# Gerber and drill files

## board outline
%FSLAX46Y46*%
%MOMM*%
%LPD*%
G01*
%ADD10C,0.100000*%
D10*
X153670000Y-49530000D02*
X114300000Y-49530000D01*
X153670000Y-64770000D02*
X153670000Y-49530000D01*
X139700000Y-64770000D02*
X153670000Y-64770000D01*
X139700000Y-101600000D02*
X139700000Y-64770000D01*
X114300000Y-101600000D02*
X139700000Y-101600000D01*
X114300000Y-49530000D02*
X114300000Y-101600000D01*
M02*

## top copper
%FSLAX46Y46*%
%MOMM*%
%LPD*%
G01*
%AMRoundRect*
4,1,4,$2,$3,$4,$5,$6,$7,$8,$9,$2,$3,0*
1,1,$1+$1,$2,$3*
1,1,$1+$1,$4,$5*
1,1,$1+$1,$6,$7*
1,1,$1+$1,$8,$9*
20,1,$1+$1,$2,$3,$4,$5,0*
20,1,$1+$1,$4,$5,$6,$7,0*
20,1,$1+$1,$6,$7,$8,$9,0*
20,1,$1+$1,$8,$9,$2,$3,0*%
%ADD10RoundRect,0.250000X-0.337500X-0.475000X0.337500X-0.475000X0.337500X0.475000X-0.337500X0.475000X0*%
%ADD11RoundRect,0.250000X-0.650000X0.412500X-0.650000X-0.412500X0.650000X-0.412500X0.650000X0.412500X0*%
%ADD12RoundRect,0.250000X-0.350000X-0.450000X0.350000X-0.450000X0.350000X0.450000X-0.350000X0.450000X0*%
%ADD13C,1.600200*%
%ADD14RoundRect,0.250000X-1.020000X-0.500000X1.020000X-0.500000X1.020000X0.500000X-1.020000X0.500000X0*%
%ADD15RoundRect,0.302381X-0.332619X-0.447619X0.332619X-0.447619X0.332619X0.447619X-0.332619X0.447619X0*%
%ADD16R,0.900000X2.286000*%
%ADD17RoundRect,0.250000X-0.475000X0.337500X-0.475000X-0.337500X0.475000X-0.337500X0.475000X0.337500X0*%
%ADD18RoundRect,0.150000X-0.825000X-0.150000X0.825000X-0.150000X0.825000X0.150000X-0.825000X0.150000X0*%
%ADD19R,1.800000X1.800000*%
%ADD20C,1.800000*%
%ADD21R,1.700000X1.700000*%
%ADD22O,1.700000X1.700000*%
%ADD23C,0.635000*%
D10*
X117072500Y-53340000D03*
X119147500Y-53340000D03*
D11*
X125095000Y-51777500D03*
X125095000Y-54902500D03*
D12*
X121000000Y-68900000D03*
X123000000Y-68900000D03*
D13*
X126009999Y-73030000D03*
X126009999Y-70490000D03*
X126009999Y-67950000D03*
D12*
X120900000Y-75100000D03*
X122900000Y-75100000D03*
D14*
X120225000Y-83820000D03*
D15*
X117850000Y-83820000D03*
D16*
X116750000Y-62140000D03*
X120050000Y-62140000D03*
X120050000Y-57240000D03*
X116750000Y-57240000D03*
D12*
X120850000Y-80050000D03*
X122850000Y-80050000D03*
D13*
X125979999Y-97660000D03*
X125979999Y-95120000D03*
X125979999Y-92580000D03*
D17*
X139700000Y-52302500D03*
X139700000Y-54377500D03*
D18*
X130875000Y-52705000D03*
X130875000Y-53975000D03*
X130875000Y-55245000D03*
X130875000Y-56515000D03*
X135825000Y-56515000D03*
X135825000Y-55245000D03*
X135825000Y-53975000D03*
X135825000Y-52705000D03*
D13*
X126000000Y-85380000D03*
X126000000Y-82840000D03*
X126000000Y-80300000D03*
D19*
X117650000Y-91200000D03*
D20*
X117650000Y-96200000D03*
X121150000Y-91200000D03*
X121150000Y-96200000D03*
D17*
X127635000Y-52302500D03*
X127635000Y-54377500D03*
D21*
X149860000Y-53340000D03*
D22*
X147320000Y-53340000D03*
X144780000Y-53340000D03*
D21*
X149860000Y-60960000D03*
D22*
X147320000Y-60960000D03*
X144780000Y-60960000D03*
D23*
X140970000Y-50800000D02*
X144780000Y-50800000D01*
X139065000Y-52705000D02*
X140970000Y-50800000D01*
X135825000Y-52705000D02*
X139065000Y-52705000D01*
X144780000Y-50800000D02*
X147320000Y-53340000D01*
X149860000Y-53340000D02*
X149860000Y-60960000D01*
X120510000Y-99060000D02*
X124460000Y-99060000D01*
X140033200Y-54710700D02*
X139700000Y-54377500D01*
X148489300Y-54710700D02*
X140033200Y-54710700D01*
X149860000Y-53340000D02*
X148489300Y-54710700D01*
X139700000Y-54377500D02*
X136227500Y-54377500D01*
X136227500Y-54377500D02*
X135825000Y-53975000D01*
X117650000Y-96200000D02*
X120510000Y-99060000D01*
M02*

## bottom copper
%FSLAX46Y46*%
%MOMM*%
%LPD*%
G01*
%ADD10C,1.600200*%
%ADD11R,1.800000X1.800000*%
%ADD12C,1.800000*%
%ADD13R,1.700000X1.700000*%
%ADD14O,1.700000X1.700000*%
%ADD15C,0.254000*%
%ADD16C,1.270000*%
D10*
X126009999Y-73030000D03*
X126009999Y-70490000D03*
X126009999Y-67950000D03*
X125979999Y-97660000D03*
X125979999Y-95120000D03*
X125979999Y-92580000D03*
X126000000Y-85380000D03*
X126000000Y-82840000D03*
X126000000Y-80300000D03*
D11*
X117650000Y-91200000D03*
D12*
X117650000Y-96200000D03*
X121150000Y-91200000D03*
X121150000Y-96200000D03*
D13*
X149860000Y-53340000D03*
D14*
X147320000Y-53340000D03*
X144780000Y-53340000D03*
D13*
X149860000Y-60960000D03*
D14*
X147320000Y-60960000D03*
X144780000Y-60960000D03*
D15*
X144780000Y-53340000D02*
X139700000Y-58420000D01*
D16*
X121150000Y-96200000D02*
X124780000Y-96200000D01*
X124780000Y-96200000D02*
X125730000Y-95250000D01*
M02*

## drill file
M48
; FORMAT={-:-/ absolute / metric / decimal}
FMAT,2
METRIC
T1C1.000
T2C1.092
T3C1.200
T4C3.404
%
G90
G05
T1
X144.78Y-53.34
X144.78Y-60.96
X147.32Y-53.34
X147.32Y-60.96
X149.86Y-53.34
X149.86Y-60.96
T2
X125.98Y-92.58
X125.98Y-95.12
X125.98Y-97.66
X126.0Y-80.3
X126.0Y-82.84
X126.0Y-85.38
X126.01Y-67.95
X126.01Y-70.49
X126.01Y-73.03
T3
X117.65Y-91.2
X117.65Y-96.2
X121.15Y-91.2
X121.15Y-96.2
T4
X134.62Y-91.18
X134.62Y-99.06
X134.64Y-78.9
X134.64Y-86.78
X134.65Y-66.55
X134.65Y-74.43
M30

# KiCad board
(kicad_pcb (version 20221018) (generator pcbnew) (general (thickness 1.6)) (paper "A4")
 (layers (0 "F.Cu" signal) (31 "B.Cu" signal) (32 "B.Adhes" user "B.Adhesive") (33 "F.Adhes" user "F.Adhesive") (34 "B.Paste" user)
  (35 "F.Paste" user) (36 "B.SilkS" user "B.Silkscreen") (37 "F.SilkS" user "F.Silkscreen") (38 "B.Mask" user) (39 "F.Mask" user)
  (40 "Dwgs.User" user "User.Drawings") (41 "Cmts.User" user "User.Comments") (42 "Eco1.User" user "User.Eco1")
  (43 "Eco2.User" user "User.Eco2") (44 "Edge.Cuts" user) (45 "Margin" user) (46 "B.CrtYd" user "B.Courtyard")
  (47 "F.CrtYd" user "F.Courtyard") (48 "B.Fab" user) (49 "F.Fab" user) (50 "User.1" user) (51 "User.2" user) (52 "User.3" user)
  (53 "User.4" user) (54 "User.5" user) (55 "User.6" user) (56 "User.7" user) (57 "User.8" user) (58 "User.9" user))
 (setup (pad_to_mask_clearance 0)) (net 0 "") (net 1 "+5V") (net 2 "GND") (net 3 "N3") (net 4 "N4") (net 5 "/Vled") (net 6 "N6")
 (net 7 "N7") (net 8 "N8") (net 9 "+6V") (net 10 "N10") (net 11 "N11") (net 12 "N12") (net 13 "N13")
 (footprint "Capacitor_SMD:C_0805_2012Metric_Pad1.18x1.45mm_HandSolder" (layer "F.Cu") (at 118.11 53.34)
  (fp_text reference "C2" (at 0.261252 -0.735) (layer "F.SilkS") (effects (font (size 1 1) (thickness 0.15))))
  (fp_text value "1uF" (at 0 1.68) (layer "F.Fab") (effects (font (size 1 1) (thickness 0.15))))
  (pad "1" smd roundrect (at -1.0375 0) (size 1.175 1.45) (layers "F.Cu" "F.Paste" "F.Mask") (roundrect_rratio 0.212766) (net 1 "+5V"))
  (pad "2" smd roundrect (at 1.0375 0) (size 1.175 1.45) (layers "F.Cu" "F.Paste" "F.Mask") (roundrect_rratio 0.212766) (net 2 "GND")))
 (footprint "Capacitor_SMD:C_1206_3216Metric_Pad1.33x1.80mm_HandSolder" (layer "F.Cu") (at 125.095 53.34 -90)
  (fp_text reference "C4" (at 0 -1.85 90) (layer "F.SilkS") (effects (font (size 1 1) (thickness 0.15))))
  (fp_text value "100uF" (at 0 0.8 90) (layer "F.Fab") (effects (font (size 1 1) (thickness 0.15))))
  (pad "1" smd roundrect (at -1.5625 0 270) (size 1.325 1.8) (layers "F.Cu" "F.Paste" "F.Mask") (roundrect_rratio 0.188679) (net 1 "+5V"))
  (pad "2" smd roundrect (at 1.5625 0 270) (size 1.325 1.8) (layers "F.Cu" "F.Paste" "F.Mask") (roundrect_rratio 0.188679) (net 2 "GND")))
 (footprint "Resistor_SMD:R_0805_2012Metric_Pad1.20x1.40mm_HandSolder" (layer "F.Cu") (at 122 68.9)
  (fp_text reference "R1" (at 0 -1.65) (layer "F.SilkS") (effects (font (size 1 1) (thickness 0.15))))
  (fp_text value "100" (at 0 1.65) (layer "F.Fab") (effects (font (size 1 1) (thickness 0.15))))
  (pad "1" smd roundrect (at -1 0) (size 1.2 1.4) (layers "F.Cu" "F.Paste" "F.Mask") (roundrect_rratio 0.208333) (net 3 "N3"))
  (pad "2" smd roundrect (at 1 0) (size 1.2 1.4) (layers "F.Cu" "F.Paste" "F.Mask") (roundrect_rratio 0.208333) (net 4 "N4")))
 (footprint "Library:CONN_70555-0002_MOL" (layer "F.Cu") (at 126.009999 73.03 90)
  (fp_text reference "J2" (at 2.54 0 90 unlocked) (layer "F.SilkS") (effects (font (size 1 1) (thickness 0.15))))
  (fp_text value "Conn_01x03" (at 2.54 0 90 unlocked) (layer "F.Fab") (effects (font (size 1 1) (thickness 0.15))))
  (pad "" np_thru_hole circle (at -1.4 8.640001 90) (size 3.4036 3.4036) (drill 3.4036) (layers "*.Cu" "*.Mask"))
  (pad "" np_thru_hole circle (at 6.48 8.640001 90) (size 3.4036 3.4036) (drill 3.4036) (layers "*.Cu" "*.Mask"))
  (pad "1" thru_hole circle (at 0 0 90) (size 1.6002 1.6002) (drill 1.0922) (layers "*.Cu" "*.Mask") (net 2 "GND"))
  (pad "2" thru_hole circle (at 2.54 0 90) (size 1.6002 1.6002) (drill 1.0922) (layers "*.Cu" "*.Mask") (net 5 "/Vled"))
  (pad "3" thru_hole circle (at 5.08 0 90) (size 1.6002 1.6002) (drill 1.0922) (layers "*.Cu" "*.Mask") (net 4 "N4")))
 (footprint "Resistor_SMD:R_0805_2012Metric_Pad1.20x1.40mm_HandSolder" (layer "F.Cu") (at 121.9 75.1)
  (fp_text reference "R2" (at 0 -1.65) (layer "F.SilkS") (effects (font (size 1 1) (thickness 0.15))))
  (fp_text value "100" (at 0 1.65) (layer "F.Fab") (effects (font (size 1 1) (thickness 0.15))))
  (pad "1" smd roundrect (at -1 0) (size 1.2 1.4) (layers "F.Cu" "F.Paste" "F.Mask") (roundrect_rratio 0.208333) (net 3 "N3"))
  (pad "2" smd roundrect (at 1 0) (size 1.2 1.4) (layers "F.Cu" "F.Paste" "F.Mask") (roundrect_rratio 0.208333) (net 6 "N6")))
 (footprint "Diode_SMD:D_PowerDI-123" (layer "F.Cu") (at 119.375 83.82 180)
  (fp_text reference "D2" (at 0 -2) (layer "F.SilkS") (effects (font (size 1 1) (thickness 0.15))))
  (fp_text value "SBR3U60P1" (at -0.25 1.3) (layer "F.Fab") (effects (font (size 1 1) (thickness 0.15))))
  (pad "1" smd roundrect (at -0.85 0) (size 2.54 1.5) (layers "F.Cu" "F.Paste" "F.Mask") (roundrect_rratio 0.1666666667) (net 5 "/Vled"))
  (pad "2" smd roundrect (at 1.525 0) (size 1.27 1.5) (layers "F.Cu" "F.Paste" "F.Mask") (roundrect_rratio 0.2380952381) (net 2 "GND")))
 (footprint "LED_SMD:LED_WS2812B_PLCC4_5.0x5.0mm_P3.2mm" (layer "F.Cu") (at 118.4 59.69 90)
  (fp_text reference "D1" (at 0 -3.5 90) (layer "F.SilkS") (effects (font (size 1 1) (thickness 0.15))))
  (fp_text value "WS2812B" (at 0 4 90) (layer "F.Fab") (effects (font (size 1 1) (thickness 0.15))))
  (pad "1" smd rect (at -2.45 -1.65 90) (size 2.286 0.9) (layers "F.Cu" "F.Paste" "F.Mask") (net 1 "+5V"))
  (pad "2" smd rect (at -2.45 1.65 90) (size 2.286 0.9) (layers "F.Cu" "F.Paste" "F.Mask") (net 3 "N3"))
  (pad "3" smd rect (at 2.45 1.65 90) (size 2.286 0.9) (layers "F.Cu" "F.Paste" "F.Mask") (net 2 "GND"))
  (pad "4" smd rect (at 2.45 -1.65 90) (size 2.286 0.9) (layers "F.Cu" "F.Paste" "F.Mask") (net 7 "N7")))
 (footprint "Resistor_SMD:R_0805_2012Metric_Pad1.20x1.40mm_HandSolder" (layer "F.Cu") (at 121.85 80.05)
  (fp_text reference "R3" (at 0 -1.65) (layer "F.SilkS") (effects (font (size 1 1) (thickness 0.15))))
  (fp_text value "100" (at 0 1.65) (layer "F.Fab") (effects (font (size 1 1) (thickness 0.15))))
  (pad "1" smd roundrect (at -1 0) (size 1.2 1.4) (layers "F.Cu" "F.Paste" "F.Mask") (roundrect_rratio 0.208333) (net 3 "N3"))
  (pad "2" smd roundrect (at 1 0) (size 1.2 1.4) (layers "F.Cu" "F.Paste" "F.Mask") (roundrect_rratio 0.208333) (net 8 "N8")))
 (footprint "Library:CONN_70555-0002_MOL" (layer "F.Cu") (at 125.979999 97.66 90)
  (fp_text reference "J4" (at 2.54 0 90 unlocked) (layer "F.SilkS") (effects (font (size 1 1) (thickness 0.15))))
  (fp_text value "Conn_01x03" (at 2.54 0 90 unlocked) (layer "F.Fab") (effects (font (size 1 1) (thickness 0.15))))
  (pad "" np_thru_hole circle (at -1.4 8.640001 90) (size 3.4036 3.4036) (drill 3.4036) (layers "*.Cu" "*.Mask"))
  (pad "" np_thru_hole circle (at 6.48 8.640001 90) (size 3.4036 3.4036) (drill 3.4036) (layers "*.Cu" "*.Mask"))
  (pad "1" thru_hole circle (at 0 0 90) (size 1.6002 1.6002) (drill 1.0922) (layers "*.Cu" "*.Mask") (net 2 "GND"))
  (pad "2" thru_hole circle (at 2.54 0 90) (size 1.6002 1.6002) (drill 1.0922) (layers "*.Cu" "*.Mask") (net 5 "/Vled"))
  (pad "3" thru_hole circle (at 5.08 0 90) (size 1.6002 1.6002) (drill 1.0922) (layers "*.Cu" "*.Mask") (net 8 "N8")))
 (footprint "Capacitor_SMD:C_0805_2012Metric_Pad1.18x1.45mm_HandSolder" (layer "F.Cu") (at 139.7 53.34 -90)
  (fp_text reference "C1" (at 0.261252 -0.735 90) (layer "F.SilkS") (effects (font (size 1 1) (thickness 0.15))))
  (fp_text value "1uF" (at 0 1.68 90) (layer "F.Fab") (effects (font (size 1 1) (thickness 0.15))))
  (pad "1" smd roundrect (at -1.0375 0 270) (size 1.175 1.45) (layers "F.Cu" "F.Paste" "F.Mask") (roundrect_rratio 0.212766) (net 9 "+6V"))
  (pad "2" smd roundrect (at 1.0375 0 270) (size 1.175 1.45) (layers "F.Cu" "F.Paste" "F.Mask") (roundrect_rratio 0.212766) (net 2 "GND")))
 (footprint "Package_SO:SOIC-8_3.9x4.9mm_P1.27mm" (layer "F.Cu") (at 133.35 54.61)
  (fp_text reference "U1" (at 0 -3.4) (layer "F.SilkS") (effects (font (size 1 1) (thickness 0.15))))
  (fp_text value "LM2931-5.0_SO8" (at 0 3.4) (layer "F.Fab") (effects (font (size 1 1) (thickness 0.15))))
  (pad "1" smd roundrect (at -2.475 -1.905) (size 1.95 0.6) (layers "F.Cu" "F.Paste" "F.Mask") (roundrect_rratio 0.25) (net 1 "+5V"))
  (pad "2" smd roundrect (at -2.475 -0.635) (size 1.95 0.6) (layers "F.Cu" "F.Paste" "F.Mask") (roundrect_rratio 0.25) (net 2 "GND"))
  (pad "3" smd roundrect (at -2.475 0.635) (size 1.95 0.6) (layers "F.Cu" "F.Paste" "F.Mask") (roundrect_rratio 0.25) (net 2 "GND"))
  (pad "4" smd roundrect (at -2.475 1.905) (size 1.95 0.6) (layers "F.Cu" "F.Paste" "F.Mask") (roundrect_rratio 0.25) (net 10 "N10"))
  (pad "5" smd roundrect (at 2.475 1.905) (size 1.95 0.6) (layers "F.Cu" "F.Paste" "F.Mask") (roundrect_rratio 0.25) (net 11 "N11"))
  (pad "6" smd roundrect (at 2.475 0.635) (size 1.95 0.6) (layers "F.Cu" "F.Paste" "F.Mask") (roundrect_rratio 0.25) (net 2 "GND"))
  (pad "7" smd roundrect (at 2.475 -0.635) (size 1.95 0.6) (layers "F.Cu" "F.Paste" "F.Mask") (roundrect_rratio 0.25) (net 2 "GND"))
  (pad "8" smd roundrect (at 2.475 -1.905) (size 1.95 0.6) (layers "F.Cu" "F.Paste" "F.Mask") (roundrect_rratio 0.25) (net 9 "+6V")))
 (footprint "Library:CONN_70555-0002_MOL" (layer "F.Cu") (at 126 85.38 90)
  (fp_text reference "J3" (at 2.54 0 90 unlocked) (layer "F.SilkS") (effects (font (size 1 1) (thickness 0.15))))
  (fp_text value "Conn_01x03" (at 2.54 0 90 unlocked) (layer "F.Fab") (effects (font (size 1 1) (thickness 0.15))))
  (pad "" np_thru_hole circle (at -1.4 8.640001 90) (size 3.4036 3.4036) (drill 3.4036) (layers "*.Cu" "*.Mask"))
  (pad "" np_thru_hole circle (at 6.48 8.640001 90) (size 3.4036 3.4036) (drill 3.4036) (layers "*.Cu" "*.Mask"))
  (pad "1" thru_hole circle (at 0 0 90) (size 1.6002 1.6002) (drill 1.0922) (layers "*.Cu" "*.Mask") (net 2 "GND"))
  (pad "2" thru_hole circle (at 2.54 0 90) (size 1.6002 1.6002) (drill 1.0922) (layers "*.Cu" "*.Mask") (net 5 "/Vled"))
  (pad "3" thru_hole circle (at 5.08 0 90) (size 1.6002 1.6002) (drill 1.0922) (layers "*.Cu" "*.Mask") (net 6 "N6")))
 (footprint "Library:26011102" (layer "F.Cu") (at 117.65 91.2)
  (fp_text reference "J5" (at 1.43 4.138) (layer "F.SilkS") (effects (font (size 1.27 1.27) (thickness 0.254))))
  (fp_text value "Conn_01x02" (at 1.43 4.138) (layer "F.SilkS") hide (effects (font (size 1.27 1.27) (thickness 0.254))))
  (pad "1" thru_hole rect (at 0 0) (size 1.8 1.8) (drill 1.2) (layers "*.Cu" "*.Mask") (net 2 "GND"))
  (pad "1" thru_hole circle (at 0 5) (size 1.8 1.8) (drill 1.2) (layers "*.Cu" "*.Mask") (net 2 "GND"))
  (pad "2" thru_hole circle (at 3.5 0) (size 1.8 1.8) (drill 1.2) (layers "*.Cu" "*.Mask") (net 5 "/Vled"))
  (pad "2" thru_hole circle (at 3.5 5) (size 1.8 1.8) (drill 1.2) (layers "*.Cu" "*.Mask") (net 5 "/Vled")))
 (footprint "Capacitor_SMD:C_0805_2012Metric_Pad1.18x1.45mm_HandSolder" (layer "F.Cu") (at 127.635 53.34 -90)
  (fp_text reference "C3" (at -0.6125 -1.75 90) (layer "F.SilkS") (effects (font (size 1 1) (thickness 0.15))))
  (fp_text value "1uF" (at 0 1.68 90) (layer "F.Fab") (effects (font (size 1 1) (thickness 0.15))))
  (pad "1" smd roundrect (at -1.0375 0 270) (size 1.175 1.45) (layers "F.Cu" "F.Paste" "F.Mask") (roundrect_rratio 0.212766) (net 1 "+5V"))
  (pad "2" smd roundrect (at 1.0375 0 270) (size 1.175 1.45) (layers "F.Cu" "F.Paste" "F.Mask") (roundrect_rratio 0.212766) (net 2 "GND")))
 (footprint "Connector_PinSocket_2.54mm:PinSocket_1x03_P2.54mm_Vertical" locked (layer "B.Cu") (at 149.86 53.34 90)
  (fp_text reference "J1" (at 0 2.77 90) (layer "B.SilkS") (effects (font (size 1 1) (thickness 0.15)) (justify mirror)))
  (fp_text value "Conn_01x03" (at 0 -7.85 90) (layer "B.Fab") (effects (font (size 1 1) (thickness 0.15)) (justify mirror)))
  (pad "1" thru_hole rect locked (at 0 0 90) (size 1.7 1.7) (drill 1) (layers "*.Cu" "*.Mask") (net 2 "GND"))
  (pad "2" thru_hole oval locked (at 0 -2.54 90) (size 1.7 1.7) (drill 1) (layers "*.Cu" "*.Mask") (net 9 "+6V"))
  (pad "3" thru_hole oval locked (at 0 -5.08 90) (size 1.7 1.7) (drill 1) (layers "*.Cu" "*.Mask") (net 7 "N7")))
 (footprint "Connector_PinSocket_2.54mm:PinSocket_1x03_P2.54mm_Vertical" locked (layer "B.Cu") (at 149.86 60.96 90)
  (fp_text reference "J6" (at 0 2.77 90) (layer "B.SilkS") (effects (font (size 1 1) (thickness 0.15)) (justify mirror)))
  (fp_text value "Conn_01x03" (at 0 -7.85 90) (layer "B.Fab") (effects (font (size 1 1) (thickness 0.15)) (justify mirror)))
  (pad "1" thru_hole rect locked (at 0 0 90) (size 1.7 1.7) (drill 1) (layers "*.Cu" "*.Mask") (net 2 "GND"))
  (pad "2" thru_hole oval locked (at 0 -2.54 90) (size 1.7 1.7) (drill 1) (layers "*.Cu" "*.Mask") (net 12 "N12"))
  (pad "3" thru_hole oval locked (at 0 -5.08 90) (size 1.7 1.7) (drill 1) (layers "*.Cu" "*.Mask") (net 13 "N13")))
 (gr_line locked (start 153.67 49.53) (end 114.3 49.53) (stroke (width 0.1) (type default)) (layer "Edge.Cuts"))
 (gr_line locked (start 153.67 64.77) (end 153.67 49.53) (stroke (width 0.1) (type default)) (layer "Edge.Cuts"))
 (gr_line locked (start 139.7 64.77) (end 153.67 64.77) (stroke (width 0.1) (type default)) (layer "Edge.Cuts"))
 (gr_line locked (start 139.7 101.6) (end 139.7 64.77) (stroke (width 0.1) (type default)) (layer "Edge.Cuts"))
 (gr_line locked (start 114.3 101.6) (end 139.7 101.6) (stroke (width 0.1) (type default)) (layer "Edge.Cuts"))
 (gr_line locked (start 114.3 49.53) (end 114.3 101.6) (stroke (width 0.1) (type default)) (layer "Edge.Cuts"))
 (segment (start 140.97 50.8) (end 144.78 50.8) (width 0.635) (layer "F.Cu") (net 9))
 (segment (start 139.065 52.705) (end 140.97 50.8) (width 0.635) (layer "F.Cu") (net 9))
 (segment (start 135.825 52.705) (end 139.065 52.705) (width 0.635) (layer "F.Cu") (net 9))
 (segment (start 144.78 50.8) (end 147.32 53.34) (width 0.635) (layer "F.Cu") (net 9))
 (segment (start 149.86 53.34) (end 149.86 60.96) (width 0.635) (layer "F.Cu") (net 2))
 (segment (start 120.51 99.06) (end 124.46 99.06) (width 0.635) (layer "F.Cu") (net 2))
 (segment (start 140.0332 54.7107) (end 139.7 54.3775) (width 0.635) (layer "F.Cu") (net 2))
 (segment (start 148.4893 54.7107) (end 140.0332 54.7107) (width 0.635) (layer "F.Cu") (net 2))
 (segment (start 149.86 53.34) (end 148.4893 54.7107) (width 0.635) (layer "F.Cu") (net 2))
 (segment (start 139.7 54.3775) (end 136.2275 54.3775) (width 0.635) (layer "F.Cu") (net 2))
 (segment (start 136.2275 54.3775) (end 135.825 53.975) (width 0.635) (layer "F.Cu") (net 2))
 (segment (start 117.65 96.2) (end 120.51 99.06) (width 0.635) (layer "F.Cu") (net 2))
 (segment (start 144.78 53.34) (end 139.7 58.42) (width 0.254) (layer "B.Cu") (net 7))
 (segment (start 121.15 96.2) (end 124.78 96.2) (width 1.27) (layer "B.Cu") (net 5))
 (segment (start 124.78 96.2) (end 125.73 95.25) (width 1.27) (layer "B.Cu") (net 5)))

